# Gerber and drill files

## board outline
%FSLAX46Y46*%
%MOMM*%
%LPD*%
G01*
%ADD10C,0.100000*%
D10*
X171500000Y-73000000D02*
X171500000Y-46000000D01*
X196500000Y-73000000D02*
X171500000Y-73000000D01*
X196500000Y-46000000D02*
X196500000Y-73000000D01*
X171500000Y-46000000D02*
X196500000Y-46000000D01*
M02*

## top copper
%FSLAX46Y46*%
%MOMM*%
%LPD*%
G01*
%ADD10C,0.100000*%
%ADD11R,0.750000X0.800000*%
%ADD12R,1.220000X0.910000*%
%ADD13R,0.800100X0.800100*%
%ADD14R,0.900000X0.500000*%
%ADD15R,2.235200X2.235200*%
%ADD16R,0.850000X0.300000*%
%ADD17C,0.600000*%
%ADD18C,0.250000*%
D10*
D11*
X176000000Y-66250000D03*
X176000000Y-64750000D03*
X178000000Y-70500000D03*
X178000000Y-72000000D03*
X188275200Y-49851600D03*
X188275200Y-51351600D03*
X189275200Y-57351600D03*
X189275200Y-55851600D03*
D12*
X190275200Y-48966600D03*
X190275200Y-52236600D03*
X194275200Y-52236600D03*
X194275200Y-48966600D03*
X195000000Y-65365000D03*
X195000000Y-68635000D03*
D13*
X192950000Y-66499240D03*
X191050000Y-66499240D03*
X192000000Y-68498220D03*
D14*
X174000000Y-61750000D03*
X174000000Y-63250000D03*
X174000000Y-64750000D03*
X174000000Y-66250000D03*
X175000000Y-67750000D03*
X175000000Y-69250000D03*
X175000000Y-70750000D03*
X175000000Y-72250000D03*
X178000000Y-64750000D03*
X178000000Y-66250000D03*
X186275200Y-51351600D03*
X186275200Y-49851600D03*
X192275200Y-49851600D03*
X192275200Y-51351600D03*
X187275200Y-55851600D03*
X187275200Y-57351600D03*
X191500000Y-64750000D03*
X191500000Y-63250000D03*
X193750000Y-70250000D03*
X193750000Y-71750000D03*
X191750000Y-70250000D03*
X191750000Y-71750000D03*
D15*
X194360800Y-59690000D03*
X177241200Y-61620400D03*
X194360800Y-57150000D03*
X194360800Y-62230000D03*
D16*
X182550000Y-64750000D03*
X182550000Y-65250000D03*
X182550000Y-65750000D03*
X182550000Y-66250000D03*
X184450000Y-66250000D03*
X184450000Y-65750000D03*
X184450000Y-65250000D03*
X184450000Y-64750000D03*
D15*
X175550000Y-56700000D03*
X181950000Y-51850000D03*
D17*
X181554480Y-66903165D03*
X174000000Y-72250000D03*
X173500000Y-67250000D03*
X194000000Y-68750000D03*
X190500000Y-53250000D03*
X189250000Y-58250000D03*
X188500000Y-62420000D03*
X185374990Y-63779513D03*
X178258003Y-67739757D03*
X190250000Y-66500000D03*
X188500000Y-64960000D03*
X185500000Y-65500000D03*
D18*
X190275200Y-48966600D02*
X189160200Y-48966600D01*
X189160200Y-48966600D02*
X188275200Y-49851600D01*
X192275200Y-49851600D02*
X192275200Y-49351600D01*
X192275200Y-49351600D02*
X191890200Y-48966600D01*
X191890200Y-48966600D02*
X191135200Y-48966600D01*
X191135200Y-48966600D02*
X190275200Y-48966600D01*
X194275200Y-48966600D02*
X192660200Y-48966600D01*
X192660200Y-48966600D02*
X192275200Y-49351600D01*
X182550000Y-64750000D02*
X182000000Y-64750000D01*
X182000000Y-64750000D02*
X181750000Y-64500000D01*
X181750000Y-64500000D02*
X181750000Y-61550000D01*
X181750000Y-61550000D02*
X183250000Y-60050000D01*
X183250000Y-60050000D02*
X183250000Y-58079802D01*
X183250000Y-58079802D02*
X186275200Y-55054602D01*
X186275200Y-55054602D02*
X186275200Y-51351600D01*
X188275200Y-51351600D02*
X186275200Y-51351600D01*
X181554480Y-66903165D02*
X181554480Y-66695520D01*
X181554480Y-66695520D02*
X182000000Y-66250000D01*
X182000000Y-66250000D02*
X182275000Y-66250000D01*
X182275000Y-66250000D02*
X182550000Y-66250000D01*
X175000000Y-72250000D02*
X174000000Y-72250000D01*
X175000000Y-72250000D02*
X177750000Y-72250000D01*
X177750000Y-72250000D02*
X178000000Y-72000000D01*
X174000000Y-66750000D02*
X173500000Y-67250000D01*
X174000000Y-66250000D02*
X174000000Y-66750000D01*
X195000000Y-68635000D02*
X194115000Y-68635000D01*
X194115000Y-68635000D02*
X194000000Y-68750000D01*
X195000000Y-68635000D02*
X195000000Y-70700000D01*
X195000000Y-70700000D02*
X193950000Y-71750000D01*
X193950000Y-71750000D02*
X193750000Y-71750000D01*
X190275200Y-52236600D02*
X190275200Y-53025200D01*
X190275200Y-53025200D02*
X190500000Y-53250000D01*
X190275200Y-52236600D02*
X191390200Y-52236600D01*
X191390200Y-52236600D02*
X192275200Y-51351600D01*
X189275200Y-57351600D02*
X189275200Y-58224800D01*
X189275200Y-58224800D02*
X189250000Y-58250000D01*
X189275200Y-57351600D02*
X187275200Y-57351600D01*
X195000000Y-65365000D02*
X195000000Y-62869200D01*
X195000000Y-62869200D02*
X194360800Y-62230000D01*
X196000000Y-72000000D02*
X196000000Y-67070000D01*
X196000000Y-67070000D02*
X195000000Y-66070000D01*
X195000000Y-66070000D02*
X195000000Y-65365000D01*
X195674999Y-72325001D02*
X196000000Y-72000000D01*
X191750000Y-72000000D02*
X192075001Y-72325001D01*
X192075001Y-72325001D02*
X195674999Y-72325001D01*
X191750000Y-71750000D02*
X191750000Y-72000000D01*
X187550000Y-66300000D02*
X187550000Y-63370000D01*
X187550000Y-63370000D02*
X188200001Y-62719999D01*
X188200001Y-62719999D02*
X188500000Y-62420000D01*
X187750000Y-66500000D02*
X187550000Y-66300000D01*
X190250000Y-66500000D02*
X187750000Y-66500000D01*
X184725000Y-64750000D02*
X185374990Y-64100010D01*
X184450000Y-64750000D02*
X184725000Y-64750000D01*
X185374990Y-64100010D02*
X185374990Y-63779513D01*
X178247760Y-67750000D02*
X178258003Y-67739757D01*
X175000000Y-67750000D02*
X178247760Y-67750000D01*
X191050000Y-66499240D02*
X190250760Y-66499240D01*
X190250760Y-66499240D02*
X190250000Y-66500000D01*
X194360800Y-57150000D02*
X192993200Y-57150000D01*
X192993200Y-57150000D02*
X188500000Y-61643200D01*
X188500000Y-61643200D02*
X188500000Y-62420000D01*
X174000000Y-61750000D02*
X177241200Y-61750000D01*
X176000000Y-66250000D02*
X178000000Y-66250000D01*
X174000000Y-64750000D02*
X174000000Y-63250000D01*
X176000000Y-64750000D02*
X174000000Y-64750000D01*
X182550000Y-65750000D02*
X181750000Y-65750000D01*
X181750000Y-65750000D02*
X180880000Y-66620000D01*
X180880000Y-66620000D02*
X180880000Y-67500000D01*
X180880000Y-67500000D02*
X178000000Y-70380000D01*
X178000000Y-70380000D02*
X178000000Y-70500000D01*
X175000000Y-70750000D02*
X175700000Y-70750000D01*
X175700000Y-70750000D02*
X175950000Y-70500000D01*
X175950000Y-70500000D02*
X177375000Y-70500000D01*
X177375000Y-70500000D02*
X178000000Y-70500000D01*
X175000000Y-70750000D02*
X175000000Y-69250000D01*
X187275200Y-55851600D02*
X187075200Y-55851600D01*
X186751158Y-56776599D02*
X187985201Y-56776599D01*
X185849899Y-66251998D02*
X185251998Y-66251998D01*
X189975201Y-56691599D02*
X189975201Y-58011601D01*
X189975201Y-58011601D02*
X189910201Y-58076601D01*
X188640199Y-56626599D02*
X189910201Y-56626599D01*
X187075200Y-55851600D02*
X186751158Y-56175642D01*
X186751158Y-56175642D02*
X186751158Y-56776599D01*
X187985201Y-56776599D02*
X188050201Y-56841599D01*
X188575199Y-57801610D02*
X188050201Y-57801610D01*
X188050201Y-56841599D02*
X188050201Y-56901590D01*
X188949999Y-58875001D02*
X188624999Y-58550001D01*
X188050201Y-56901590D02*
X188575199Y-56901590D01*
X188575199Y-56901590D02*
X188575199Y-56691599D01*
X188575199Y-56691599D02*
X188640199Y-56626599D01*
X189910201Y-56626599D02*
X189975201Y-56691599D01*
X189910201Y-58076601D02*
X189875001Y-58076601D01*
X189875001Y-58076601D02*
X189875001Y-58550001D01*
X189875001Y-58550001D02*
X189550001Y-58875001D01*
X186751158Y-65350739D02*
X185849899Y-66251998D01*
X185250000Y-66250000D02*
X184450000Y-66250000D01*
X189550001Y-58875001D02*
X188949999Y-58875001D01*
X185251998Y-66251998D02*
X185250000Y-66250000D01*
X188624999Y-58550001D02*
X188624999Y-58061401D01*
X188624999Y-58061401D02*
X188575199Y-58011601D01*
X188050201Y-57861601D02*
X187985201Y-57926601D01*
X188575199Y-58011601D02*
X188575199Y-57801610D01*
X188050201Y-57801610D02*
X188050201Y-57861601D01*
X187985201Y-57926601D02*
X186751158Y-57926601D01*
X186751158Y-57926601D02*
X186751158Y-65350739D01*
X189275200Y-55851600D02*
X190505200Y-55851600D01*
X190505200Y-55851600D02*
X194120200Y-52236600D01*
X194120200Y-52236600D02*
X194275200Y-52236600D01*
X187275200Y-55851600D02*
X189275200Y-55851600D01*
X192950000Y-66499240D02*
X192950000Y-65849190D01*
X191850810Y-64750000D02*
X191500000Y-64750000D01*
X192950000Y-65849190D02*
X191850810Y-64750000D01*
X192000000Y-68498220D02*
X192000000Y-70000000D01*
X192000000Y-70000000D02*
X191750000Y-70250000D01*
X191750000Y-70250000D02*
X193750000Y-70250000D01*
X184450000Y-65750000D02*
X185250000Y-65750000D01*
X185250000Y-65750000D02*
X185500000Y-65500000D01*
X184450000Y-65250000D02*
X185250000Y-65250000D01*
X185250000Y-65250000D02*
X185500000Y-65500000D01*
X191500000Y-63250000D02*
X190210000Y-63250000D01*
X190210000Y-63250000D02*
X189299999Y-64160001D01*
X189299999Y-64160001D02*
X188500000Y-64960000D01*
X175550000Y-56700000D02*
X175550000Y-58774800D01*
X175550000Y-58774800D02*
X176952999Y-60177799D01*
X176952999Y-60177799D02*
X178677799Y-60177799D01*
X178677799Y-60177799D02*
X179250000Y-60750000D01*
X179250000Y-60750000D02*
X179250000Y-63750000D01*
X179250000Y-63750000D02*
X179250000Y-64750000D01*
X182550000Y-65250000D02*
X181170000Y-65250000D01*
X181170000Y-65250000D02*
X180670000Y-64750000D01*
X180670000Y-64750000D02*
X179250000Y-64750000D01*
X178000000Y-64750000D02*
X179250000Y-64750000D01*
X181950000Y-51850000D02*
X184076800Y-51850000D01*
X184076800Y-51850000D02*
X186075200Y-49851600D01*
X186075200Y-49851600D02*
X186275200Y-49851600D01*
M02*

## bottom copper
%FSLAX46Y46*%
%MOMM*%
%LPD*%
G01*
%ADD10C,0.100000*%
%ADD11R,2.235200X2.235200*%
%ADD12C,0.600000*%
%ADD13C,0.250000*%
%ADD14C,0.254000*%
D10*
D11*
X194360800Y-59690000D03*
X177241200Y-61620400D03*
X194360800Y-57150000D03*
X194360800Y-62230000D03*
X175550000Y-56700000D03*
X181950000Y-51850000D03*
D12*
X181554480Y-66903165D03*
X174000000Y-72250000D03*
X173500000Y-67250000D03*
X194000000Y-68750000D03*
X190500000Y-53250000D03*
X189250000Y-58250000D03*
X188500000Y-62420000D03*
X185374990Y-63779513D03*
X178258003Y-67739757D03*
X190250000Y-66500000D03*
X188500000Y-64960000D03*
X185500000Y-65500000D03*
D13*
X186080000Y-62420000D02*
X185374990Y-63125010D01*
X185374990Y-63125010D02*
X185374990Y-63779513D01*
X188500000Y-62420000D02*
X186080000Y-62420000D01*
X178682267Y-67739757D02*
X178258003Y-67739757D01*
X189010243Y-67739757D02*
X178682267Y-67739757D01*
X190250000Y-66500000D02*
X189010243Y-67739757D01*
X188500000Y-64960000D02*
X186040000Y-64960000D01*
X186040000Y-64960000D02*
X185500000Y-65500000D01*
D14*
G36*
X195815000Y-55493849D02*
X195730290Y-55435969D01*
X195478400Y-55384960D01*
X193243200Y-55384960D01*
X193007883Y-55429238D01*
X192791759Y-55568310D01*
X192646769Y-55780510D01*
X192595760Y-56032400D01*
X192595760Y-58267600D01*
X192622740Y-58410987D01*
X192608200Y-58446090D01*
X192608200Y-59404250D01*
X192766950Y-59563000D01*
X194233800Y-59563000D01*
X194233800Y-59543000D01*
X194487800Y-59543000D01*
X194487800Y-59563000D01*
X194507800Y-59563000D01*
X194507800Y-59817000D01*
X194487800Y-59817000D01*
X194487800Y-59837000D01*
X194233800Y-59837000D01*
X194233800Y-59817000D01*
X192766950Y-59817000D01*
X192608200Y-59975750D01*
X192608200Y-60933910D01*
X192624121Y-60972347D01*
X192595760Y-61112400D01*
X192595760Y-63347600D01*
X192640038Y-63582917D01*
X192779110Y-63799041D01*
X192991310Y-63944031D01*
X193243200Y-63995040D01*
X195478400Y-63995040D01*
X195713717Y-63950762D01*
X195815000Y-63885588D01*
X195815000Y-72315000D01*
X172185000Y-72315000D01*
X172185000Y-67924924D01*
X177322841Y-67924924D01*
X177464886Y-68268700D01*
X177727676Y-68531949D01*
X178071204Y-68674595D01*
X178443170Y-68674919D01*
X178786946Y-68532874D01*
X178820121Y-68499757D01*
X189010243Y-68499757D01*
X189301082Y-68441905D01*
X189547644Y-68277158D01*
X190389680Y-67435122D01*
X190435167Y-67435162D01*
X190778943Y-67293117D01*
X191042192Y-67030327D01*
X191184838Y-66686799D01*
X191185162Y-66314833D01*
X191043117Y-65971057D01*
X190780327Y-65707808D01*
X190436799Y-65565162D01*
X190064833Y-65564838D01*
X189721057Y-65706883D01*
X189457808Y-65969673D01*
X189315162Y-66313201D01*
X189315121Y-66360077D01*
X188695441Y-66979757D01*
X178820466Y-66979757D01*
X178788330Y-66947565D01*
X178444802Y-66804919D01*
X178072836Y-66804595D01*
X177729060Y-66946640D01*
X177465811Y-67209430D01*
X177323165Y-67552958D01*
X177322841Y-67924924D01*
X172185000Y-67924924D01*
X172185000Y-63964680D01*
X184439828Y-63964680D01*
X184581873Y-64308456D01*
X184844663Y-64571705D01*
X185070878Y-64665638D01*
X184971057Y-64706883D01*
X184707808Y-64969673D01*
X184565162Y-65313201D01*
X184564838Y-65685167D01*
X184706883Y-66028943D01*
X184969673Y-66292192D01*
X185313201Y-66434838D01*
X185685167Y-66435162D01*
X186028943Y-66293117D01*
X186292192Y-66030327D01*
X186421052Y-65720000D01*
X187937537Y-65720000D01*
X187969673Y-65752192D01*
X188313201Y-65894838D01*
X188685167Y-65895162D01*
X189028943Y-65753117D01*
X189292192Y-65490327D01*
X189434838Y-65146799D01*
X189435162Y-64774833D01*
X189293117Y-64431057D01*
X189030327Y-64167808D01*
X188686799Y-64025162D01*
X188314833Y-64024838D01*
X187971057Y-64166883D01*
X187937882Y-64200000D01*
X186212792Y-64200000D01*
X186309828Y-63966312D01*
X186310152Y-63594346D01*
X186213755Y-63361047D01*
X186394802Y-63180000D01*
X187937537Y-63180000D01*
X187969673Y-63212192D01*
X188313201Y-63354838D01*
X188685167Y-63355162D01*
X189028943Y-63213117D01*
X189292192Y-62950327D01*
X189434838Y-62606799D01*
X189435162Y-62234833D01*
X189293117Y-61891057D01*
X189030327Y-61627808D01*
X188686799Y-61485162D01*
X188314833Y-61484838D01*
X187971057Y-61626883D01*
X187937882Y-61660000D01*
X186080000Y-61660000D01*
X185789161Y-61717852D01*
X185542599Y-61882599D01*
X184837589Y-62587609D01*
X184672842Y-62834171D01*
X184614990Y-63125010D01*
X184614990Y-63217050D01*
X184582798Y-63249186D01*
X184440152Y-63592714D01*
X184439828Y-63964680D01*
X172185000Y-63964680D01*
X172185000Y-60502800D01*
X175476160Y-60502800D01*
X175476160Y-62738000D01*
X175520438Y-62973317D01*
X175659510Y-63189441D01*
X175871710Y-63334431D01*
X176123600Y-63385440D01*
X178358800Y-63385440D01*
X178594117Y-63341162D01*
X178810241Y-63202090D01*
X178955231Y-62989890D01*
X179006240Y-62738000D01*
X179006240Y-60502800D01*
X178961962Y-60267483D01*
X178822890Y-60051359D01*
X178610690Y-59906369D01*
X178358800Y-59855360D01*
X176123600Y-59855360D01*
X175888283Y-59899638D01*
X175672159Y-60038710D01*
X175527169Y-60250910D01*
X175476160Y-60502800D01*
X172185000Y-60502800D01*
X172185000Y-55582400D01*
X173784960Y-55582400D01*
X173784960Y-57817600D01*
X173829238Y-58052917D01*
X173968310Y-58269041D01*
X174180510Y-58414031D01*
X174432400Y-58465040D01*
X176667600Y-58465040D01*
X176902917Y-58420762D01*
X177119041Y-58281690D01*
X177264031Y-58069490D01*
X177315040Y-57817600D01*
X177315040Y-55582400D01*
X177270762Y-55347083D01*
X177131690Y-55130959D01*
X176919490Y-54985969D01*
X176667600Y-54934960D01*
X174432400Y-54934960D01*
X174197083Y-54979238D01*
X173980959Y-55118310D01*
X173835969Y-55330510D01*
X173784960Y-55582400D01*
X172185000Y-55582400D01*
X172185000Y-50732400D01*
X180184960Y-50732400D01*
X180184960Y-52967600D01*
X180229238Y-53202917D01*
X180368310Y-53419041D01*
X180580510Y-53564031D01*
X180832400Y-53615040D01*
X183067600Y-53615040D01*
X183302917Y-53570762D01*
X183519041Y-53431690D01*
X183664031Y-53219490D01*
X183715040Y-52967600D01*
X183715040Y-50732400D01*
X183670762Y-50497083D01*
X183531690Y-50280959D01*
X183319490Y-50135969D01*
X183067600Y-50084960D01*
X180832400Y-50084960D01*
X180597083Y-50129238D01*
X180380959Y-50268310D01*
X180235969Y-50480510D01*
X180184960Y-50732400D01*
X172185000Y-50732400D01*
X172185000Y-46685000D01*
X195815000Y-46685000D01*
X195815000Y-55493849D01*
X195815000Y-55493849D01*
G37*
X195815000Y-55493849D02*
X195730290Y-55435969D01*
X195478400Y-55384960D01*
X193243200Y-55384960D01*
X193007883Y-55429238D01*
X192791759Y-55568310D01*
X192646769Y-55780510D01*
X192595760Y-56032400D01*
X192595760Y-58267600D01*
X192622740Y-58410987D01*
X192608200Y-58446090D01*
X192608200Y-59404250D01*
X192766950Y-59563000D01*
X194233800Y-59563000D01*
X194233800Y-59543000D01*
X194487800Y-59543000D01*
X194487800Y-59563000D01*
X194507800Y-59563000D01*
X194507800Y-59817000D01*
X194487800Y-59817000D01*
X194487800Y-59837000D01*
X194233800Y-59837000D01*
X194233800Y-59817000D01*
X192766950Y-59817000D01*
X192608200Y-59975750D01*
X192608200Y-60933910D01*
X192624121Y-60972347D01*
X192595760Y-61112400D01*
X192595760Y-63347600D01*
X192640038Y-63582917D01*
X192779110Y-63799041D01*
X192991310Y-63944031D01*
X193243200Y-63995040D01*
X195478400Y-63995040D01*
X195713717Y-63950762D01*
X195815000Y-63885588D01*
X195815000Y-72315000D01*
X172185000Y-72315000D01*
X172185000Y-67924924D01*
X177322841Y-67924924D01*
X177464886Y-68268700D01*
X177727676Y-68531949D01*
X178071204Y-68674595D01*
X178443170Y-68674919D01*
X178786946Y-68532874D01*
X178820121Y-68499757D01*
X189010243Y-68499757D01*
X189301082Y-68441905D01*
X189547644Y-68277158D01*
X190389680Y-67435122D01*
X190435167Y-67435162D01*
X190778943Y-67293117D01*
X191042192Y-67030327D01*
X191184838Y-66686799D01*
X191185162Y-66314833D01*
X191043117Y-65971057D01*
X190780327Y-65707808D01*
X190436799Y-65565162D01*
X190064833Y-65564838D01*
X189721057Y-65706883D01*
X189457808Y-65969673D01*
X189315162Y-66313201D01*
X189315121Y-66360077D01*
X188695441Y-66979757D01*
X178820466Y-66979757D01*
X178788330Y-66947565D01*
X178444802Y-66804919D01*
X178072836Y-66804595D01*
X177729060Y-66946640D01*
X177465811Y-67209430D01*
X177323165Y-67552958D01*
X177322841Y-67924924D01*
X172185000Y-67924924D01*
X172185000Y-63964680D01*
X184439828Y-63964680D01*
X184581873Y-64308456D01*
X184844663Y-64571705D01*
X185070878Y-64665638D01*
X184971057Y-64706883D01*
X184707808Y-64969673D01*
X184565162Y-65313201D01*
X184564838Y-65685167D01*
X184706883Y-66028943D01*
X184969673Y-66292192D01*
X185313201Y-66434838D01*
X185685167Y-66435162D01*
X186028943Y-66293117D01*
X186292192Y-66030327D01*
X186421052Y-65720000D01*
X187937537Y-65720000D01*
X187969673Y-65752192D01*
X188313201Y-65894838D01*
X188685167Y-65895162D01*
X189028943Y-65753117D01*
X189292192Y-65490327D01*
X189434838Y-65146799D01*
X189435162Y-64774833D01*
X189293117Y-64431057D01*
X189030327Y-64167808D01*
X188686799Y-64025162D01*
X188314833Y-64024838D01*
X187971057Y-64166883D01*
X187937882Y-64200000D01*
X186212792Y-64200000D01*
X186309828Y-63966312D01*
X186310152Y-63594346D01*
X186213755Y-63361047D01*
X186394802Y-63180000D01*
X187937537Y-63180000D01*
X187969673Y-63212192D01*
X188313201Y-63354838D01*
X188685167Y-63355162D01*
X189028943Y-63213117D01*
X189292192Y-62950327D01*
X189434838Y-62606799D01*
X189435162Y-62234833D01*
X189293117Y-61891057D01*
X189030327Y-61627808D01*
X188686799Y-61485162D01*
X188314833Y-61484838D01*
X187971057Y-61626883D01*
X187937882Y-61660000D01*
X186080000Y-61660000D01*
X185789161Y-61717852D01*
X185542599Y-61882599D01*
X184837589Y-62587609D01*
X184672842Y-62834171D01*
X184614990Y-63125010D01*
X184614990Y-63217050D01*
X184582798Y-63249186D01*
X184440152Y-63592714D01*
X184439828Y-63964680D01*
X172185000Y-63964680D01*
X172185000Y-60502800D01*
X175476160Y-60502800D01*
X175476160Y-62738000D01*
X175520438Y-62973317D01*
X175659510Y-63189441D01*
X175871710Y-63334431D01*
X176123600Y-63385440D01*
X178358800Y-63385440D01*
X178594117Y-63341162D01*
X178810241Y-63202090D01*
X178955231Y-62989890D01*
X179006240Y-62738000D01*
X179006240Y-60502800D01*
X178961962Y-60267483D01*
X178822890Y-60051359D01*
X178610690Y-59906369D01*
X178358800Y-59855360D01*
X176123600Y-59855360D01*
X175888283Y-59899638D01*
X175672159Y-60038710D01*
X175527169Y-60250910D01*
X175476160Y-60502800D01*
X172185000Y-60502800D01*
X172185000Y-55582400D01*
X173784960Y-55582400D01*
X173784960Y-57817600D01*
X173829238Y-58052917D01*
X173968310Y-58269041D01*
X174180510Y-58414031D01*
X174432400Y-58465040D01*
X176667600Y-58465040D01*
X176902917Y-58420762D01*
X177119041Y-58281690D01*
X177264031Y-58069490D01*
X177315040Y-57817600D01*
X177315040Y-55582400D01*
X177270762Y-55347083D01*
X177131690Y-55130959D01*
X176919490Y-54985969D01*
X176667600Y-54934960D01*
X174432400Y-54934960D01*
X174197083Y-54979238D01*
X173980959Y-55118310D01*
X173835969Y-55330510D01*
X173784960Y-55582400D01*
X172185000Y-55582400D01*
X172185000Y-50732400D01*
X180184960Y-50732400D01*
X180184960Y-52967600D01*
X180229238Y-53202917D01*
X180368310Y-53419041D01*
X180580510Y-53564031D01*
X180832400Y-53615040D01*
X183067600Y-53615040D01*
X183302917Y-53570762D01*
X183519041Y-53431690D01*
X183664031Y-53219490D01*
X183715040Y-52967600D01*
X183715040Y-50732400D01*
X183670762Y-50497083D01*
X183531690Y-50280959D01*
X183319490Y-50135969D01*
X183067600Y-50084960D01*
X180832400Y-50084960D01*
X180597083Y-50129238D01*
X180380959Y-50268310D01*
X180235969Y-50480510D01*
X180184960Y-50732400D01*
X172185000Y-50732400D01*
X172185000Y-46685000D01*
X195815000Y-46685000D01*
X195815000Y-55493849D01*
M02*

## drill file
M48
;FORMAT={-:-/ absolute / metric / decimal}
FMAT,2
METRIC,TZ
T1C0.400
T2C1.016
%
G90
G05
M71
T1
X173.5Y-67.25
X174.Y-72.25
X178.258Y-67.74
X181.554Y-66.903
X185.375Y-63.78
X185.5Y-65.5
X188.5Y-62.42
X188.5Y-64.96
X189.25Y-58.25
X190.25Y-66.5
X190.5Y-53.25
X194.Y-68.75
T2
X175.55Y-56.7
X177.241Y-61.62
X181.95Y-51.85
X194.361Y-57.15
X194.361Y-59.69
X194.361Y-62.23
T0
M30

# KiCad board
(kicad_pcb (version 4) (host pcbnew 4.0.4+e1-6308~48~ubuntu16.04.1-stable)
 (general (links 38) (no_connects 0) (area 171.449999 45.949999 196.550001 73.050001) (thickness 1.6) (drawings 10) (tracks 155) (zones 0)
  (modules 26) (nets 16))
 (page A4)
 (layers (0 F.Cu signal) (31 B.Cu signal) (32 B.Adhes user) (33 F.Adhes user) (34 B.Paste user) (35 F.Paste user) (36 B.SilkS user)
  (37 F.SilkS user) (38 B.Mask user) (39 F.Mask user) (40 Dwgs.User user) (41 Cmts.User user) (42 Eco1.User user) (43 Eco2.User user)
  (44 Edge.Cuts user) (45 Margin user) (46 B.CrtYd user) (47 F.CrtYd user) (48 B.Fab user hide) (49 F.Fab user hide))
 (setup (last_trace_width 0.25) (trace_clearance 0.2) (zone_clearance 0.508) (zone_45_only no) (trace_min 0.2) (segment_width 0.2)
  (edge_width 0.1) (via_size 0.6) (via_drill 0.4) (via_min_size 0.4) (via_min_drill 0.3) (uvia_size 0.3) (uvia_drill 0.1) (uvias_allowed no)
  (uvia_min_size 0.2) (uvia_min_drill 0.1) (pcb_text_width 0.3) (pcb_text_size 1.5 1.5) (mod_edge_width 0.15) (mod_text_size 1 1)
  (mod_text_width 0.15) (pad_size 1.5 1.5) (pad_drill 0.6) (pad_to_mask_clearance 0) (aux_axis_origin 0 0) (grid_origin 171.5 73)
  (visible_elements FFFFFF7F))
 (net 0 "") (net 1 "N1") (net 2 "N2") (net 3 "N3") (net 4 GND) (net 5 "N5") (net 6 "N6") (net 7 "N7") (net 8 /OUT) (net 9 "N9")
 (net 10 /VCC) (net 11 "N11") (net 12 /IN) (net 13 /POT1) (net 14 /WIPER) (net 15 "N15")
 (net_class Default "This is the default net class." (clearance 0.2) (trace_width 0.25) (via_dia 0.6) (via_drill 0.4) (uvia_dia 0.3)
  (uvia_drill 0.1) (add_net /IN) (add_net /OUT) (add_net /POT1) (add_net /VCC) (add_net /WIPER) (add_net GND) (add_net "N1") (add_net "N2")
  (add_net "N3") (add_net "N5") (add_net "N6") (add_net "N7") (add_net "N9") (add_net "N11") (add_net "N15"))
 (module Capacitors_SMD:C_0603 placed (layer F.Cu) (at 176 65.5 90)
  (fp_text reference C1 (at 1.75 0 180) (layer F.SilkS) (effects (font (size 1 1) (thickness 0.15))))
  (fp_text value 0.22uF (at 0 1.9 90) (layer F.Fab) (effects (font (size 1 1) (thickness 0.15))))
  (pad 1 smd rect (at -0.75 0 90) (size 0.8 0.75) (layers F.Cu F.Paste F.Mask) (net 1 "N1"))
  (pad 2 smd rect (at 0.75 0 90) (size 0.8 0.75) (layers F.Cu F.Paste F.Mask) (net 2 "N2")))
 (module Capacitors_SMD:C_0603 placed (layer F.Cu) (at 178 71.25 270)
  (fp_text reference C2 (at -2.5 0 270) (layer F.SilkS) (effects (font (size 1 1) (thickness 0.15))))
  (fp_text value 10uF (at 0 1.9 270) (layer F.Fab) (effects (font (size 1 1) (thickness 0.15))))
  (pad 1 smd rect (at -0.75 0 270) (size 0.8 0.75) (layers F.Cu F.Paste F.Mask) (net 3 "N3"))
  (pad 2 smd rect (at 0.75 0 270) (size 0.8 0.75) (layers F.Cu F.Paste F.Mask) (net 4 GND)))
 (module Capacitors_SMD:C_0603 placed (layer F.Cu) (at 188.2752 50.6016 270)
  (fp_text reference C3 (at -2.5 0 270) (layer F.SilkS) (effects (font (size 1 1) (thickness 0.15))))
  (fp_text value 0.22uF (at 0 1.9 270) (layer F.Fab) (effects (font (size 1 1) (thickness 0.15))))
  (pad 1 smd rect (at -0.75 0 270) (size 0.8 0.75) (layers F.Cu F.Paste F.Mask) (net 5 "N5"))
  (pad 2 smd rect (at 0.75 0 270) (size 0.8 0.75) (layers F.Cu F.Paste F.Mask) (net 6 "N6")))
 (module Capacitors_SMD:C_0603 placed (layer F.Cu) (at 189.2752 56.6016 90)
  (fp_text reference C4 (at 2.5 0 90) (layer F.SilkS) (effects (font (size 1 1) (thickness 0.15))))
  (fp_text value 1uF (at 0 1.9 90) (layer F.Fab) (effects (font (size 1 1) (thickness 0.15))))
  (pad 1 smd rect (at -0.75 0 90) (size 0.8 0.75) (layers F.Cu F.Paste F.Mask) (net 4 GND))
  (pad 2 smd rect (at 0.75 0 90) (size 0.8 0.75) (layers F.Cu F.Paste F.Mask) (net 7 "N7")))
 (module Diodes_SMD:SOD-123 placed (layer F.Cu) (at 190.2752 50.6016 270)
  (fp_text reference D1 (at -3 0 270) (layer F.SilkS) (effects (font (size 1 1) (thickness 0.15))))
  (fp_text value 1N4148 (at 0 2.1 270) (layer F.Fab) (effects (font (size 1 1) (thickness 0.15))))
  (pad 1 smd rect (at -1.635 0 270) (size 0.91 1.22) (layers F.Cu F.Paste F.Mask) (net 5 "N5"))
  (pad 2 smd rect (at 1.635 0 270) (size 0.91 1.22) (layers F.Cu F.Paste F.Mask) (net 4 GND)))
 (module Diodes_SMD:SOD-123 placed (layer F.Cu) (at 194.2752 50.6016 90)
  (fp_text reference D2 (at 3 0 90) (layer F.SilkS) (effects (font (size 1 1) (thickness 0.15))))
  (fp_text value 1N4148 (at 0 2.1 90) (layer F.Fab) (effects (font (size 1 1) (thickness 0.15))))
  (pad 1 smd rect (at -1.635 0 90) (size 0.91 1.22) (layers F.Cu F.Paste F.Mask) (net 7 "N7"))
  (pad 2 smd rect (at 1.635 0 90) (size 0.91 1.22) (layers F.Cu F.Paste F.Mask) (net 5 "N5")))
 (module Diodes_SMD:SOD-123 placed (layer F.Cu) (at 195 67 270)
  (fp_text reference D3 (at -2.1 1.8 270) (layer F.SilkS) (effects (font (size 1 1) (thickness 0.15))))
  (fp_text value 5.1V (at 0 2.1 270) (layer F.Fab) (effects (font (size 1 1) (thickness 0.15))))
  (pad 1 smd rect (at -1.635 0 270) (size 0.91 1.22) (layers F.Cu F.Paste F.Mask) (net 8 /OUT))
  (pad 2 smd rect (at 1.635 0 270) (size 0.91 1.22) (layers F.Cu F.Paste F.Mask) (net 4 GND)))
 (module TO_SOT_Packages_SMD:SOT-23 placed (layer F.Cu) (at 192 67.5 180)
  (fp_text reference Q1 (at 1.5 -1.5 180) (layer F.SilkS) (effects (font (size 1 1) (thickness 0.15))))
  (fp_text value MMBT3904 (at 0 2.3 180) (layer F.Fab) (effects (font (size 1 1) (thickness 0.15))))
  (pad 1 smd rect (at -0.95 1.00076 180) (size 0.8001 0.8001) (layers F.Cu F.Paste F.Mask) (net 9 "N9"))
  (pad 2 smd rect (at 0.95 1.00076 180) (size 0.8001 0.8001) (layers F.Cu F.Paste F.Mask) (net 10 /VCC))
  (pad 3 smd rect (at 0 -0.99822 180) (size 0.8001 0.8001) (layers F.Cu F.Paste F.Mask) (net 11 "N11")))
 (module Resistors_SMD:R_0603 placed (layer F.Cu) (at 174 62.5 270)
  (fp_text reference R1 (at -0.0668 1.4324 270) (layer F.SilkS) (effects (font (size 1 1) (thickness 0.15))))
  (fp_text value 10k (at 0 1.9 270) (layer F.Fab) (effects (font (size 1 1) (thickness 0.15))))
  (pad 1 smd rect (at -0.75 0 270) (size 0.5 0.9) (layers F.Cu F.Paste F.Mask) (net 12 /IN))
  (pad 2 smd rect (at 0.75 0 270) (size 0.5 0.9) (layers F.Cu F.Paste F.Mask) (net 2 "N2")))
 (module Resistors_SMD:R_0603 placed (layer F.Cu) (at 174 65.5 270)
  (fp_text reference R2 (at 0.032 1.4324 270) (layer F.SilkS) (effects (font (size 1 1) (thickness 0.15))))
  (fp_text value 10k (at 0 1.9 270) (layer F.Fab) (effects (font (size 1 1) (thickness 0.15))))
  (pad 1 smd rect (at -0.75 0 270) (size 0.5 0.9) (layers F.Cu F.Paste F.Mask) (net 2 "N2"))
  (pad 2 smd rect (at 0.75 0 270) (size 0.5 0.9) (layers F.Cu F.Paste F.Mask) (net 4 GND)))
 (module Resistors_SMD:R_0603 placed (layer F.Cu) (at 175 68.5 270)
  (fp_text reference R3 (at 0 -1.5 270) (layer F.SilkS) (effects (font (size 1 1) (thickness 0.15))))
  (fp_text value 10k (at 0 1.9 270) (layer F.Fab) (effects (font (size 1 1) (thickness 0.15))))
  (pad 1 smd rect (at -0.75 0 270) (size 0.5 0.9) (layers F.Cu F.Paste F.Mask) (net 10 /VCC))
  (pad 2 smd rect (at 0.75 0 270) (size 0.5 0.9) (layers F.Cu F.Paste F.Mask) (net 3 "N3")))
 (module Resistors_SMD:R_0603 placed (layer F.Cu) (at 175 71.5 270)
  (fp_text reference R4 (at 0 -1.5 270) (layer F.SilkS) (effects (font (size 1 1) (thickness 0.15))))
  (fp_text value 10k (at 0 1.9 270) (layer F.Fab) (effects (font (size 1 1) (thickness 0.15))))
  (pad 1 smd rect (at -0.75 0 270) (size 0.5 0.9) (layers F.Cu F.Paste F.Mask) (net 3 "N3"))
  (pad 2 smd rect (at 0.75 0 270) (size 0.5 0.9) (layers F.Cu F.Paste F.Mask) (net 4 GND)))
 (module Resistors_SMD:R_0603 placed (layer F.Cu) (at 178 65.5 270)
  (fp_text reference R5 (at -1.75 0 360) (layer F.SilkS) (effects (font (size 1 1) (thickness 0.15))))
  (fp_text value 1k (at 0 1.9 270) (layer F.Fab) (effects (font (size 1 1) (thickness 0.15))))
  (pad 1 smd rect (at -0.75 0 270) (size 0.5 0.9) (layers F.Cu F.Paste F.Mask) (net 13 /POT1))
  (pad 2 smd rect (at 0.75 0 270) (size 0.5 0.9) (layers F.Cu F.Paste F.Mask) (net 1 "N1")))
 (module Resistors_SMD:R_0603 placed (layer F.Cu) (at 186.2752 50.6016 90)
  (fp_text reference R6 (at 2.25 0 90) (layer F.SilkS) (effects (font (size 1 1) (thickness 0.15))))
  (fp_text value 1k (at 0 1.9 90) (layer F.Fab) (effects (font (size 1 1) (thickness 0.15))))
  (pad 1 smd rect (at -0.75 0 90) (size 0.5 0.9) (layers F.Cu F.Paste F.Mask) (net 6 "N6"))
  (pad 2 smd rect (at 0.75 0 90) (size 0.5 0.9) (layers F.Cu F.Paste F.Mask) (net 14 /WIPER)))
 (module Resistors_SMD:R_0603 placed (layer F.Cu) (at 192.2752 50.6016 270)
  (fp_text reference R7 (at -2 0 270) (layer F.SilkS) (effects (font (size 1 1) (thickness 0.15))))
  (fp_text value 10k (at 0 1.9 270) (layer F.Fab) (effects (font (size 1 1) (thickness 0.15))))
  (pad 1 smd rect (at -0.75 0 270) (size 0.5 0.9) (layers F.Cu F.Paste F.Mask) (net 5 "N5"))
  (pad 2 smd rect (at 0.75 0 270) (size 0.5 0.9) (layers F.Cu F.Paste F.Mask) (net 4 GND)))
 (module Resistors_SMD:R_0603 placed (layer F.Cu) (at 187.2752 56.6016 270)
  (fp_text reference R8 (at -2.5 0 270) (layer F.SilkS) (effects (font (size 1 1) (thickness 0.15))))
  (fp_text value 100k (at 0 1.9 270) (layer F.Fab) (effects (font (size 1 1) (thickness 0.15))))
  (pad 1 smd rect (at -0.75 0 270) (size 0.5 0.9) (layers F.Cu F.Paste F.Mask) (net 7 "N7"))
  (pad 2 smd rect (at 0.75 0 270) (size 0.5 0.9) (layers F.Cu F.Paste F.Mask) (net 4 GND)))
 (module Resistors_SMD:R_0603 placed (layer F.Cu) (at 191.5 64 90)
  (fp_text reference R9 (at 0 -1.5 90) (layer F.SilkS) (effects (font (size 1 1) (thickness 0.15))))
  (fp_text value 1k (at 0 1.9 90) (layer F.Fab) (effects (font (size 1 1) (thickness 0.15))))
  (pad 1 smd rect (at -0.75 0 90) (size 0.5 0.9) (layers F.Cu F.Paste F.Mask) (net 9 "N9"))
  (pad 2 smd rect (at 0.75 0 90) (size 0.5 0.9) (layers F.Cu F.Paste F.Mask) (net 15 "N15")))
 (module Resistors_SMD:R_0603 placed (layer F.Cu) (at 193.75 71 270)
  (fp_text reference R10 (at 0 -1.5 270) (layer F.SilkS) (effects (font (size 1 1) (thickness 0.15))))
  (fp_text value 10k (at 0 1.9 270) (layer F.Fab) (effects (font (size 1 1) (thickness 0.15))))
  (pad 1 smd rect (at -0.75 0 270) (size 0.5 0.9) (layers F.Cu F.Paste F.Mask) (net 11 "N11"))
  (pad 2 smd rect (at 0.75 0 270) (size 0.5 0.9) (layers F.Cu F.Paste F.Mask) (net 4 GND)))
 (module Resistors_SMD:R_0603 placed (layer F.Cu) (at 191.75 71 270)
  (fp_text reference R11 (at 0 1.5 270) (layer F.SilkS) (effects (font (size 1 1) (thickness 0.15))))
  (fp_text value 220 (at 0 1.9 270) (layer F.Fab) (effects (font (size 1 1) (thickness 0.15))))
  (pad 1 smd rect (at -0.75 0 270) (size 0.5 0.9) (layers F.Cu F.Paste F.Mask) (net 11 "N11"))
  (pad 2 smd rect (at 0.75 0 270) (size 0.5 0.9) (layers F.Cu F.Paste F.Mask) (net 8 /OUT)))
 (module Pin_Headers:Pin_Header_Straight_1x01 (layer F.Cu) (at 194.3608 59.69)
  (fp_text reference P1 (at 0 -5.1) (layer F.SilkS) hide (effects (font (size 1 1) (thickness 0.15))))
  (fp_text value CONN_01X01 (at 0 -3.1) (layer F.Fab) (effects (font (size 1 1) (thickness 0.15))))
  (pad 1 thru_hole rect (at 0 0) (size 2.2352 2.2352) (drill 1.016) (layers *.Cu *.Mask F.SilkS) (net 4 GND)))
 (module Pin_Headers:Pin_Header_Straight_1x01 (layer F.Cu) (at 177.2412 61.6204)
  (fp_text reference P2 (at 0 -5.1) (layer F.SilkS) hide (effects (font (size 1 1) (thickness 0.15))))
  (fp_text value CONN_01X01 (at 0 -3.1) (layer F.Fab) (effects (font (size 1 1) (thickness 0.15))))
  (pad 1 thru_hole rect (at 0 0) (size 2.2352 2.2352) (drill 1.016) (layers *.Cu *.Mask F.SilkS) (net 12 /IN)))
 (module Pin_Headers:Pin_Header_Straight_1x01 (layer F.Cu) (at 194.3608 57.15)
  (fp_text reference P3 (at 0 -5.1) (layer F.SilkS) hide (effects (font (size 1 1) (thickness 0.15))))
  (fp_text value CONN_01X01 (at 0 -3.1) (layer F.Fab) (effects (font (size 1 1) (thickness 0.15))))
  (pad 1 thru_hole rect (at 0 0) (size 2.2352 2.2352) (drill 1.016) (layers *.Cu *.Mask F.SilkS) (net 10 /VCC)))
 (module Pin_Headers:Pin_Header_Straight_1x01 (layer F.Cu) (at 194.3608 62.23)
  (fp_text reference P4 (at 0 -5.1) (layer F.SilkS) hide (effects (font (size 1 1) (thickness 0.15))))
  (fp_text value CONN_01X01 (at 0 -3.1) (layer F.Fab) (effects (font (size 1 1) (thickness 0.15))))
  (pad 1 thru_hole rect (at 0 0) (size 2.2352 2.2352) (drill 1.016) (layers *.Cu *.Mask F.SilkS) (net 8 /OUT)))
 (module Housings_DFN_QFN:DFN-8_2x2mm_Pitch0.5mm (layer F.Cu) (at 183.5 65.5)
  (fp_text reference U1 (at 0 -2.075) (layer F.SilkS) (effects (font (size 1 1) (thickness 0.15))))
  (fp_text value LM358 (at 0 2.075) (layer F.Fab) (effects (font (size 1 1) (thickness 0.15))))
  (pad 1 smd rect (at -0.95 -0.75) (size 0.85 0.3) (layers F.Cu F.Paste F.Mask) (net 6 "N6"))
  (pad 2 smd rect (at -0.95 -0.25) (size 0.85 0.3) (layers F.Cu F.Paste F.Mask) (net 13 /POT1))
  (pad 3 smd rect (at -0.95 0.25) (size 0.85 0.3) (layers F.Cu F.Paste F.Mask) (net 3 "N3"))
  (pad 4 smd rect (at -0.95 0.75) (size 0.85 0.3) (layers F.Cu F.Paste F.Mask) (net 4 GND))
  (pad 5 smd rect (at 0.95 0.75) (size 0.85 0.3) (layers F.Cu F.Paste F.Mask) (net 7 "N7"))
  (pad 6 smd rect (at 0.95 0.25) (size 0.85 0.3) (layers F.Cu F.Paste F.Mask) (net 15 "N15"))
  (pad 7 smd rect (at 0.95 -0.25) (size 0.85 0.3) (layers F.Cu F.Paste F.Mask) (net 15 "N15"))
  (pad 8 smd rect (at 0.95 -0.75) (size 0.85 0.3) (layers F.Cu F.Paste F.Mask) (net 10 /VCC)))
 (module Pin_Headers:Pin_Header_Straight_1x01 (layer F.Cu) (at 175.55 56.7)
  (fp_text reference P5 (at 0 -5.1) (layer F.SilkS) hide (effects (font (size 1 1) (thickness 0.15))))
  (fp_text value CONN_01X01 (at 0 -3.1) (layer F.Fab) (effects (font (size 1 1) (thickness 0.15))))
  (pad 1 thru_hole rect (at 0 0) (size 2.2352 2.2352) (drill 1.016) (layers *.Cu *.Mask F.SilkS) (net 13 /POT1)))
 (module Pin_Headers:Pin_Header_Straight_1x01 (layer F.Cu) (at 181.95 51.85)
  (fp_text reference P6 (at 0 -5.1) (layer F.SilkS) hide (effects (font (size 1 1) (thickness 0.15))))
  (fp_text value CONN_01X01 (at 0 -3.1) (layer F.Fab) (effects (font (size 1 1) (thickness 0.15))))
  (pad 1 thru_hole rect (at 0 0) (size 2.2352 2.2352) (drill 1.016) (layers *.Cu *.Mask F.SilkS) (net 14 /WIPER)))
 (gr_line (start 171.5 73) (end 171.5 46) (layer Edge.Cuts) (width 0.1))
 (gr_line (start 196.5 73) (end 171.5 73) (layer Edge.Cuts) (width 0.1))
 (gr_line (start 196.5 46) (end 196.5 73) (layer Edge.Cuts) (width 0.1))
 (gr_line (start 171.5 46) (end 196.5 46) (layer Edge.Cuts) (width 0.1))
 (segment (start 190.2752 48.9666) (end 189.1602 48.9666) (width 0.25) (layer F.Cu) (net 5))
 (segment (start 189.1602 48.9666) (end 188.2752 49.8516) (width 0.25) (layer F.Cu) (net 5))
 (segment (start 192.2752 49.8516) (end 192.2752 49.3516) (width 0.25) (layer F.Cu) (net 5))
 (segment (start 192.2752 49.3516) (end 191.8902 48.9666) (width 0.25) (layer F.Cu) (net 5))
 (segment (start 191.8902 48.9666) (end 191.1352 48.9666) (width 0.25) (layer F.Cu) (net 5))
 (segment (start 191.1352 48.9666) (end 190.2752 48.9666) (width 0.25) (layer F.Cu) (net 5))
 (segment (start 194.2752 48.9666) (end 192.6602 48.9666) (width 0.25) (layer F.Cu) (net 5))
 (segment (start 192.6602 48.9666) (end 192.2752 49.3516) (width 0.25) (layer F.Cu) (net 5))
 (segment (start 182.55 64.75) (end 182 64.75) (width 0.25) (layer F.Cu) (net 6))
 (segment (start 182 64.75) (end 181.75 64.5) (width 0.25) (layer F.Cu) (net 6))
 (segment (start 181.75 64.5) (end 181.75 61.55) (width 0.25) (layer F.Cu) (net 6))
 (segment (start 181.75 61.55) (end 183.25 60.05) (width 0.25) (layer F.Cu) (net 6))
 (segment (start 183.25 60.05) (end 183.25 58.079802) (width 0.25) (layer F.Cu) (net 6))
 (segment (start 183.25 58.079802) (end 186.2752 55.054602) (width 0.25) (layer F.Cu) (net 6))
 (segment (start 186.2752 55.054602) (end 186.2752 51.3516) (width 0.25) (layer F.Cu) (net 6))
 (segment (start 188.2752 51.3516) (end 186.2752 51.3516) (width 0.25) (layer F.Cu) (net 6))
 (via (at 181.55448 66.903165) (size 0.6) (drill 0.4) (layers F.Cu B.Cu) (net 4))
 (segment (start 181.55448 66.903165) (end 181.55448 66.69552) (width 0.25) (layer F.Cu) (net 4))
 (segment (start 181.55448 66.69552) (end 182 66.25) (width 0.25) (layer F.Cu) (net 4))
 (segment (start 182 66.25) (end 182.275 66.25) (width 0.25) (layer F.Cu) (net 4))
 (segment (start 182.275 66.25) (end 182.55 66.25) (width 0.25) (layer F.Cu) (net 4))
 (segment (start 175 72.25) (end 174 72.25) (width 0.25) (layer F.Cu) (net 4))
 (via (at 174 72.25) (size 0.6) (drill 0.4) (layers F.Cu B.Cu) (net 4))
 (segment (start 175 72.25) (end 177.75 72.25) (width 0.25) (layer F.Cu) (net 4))
 (segment (start 177.75 72.25) (end 178 72) (width 0.25) (layer F.Cu) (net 4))
 (segment (start 174 66.75) (end 173.5 67.25) (width 0.25) (layer F.Cu) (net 4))
 (via (at 173.5 67.25) (size 0.6) (drill 0.4) (layers F.Cu B.Cu) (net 4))
 (segment (start 174 66.25) (end 174 66.75) (width 0.25) (layer F.Cu) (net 4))
 (segment (start 195 68.635) (end 194.115 68.635) (width 0.25) (layer F.Cu) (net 4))
 (segment (start 194.115 68.635) (end 194 68.75) (width 0.25) (layer F.Cu) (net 4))
 (via (at 194 68.75) (size 0.6) (drill 0.4) (layers F.Cu B.Cu) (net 4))
 (segment (start 195 68.635) (end 195 70.7) (width 0.25) (layer F.Cu) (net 4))
 (segment (start 195 70.7) (end 193.95 71.75) (width 0.25) (layer F.Cu) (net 4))
 (segment (start 193.95 71.75) (end 193.75 71.75) (width 0.25) (layer F.Cu) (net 4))
 (segment (start 190.2752 52.2366) (end 190.2752 53.0252) (width 0.25) (layer F.Cu) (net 4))
 (segment (start 190.2752 53.0252) (end 190.5 53.25) (width 0.25) (layer F.Cu) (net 4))
 (via (at 190.5 53.25) (size 0.6) (drill 0.4) (layers F.Cu B.Cu) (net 4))
 (segment (start 190.2752 52.2366) (end 191.3902 52.2366) (width 0.25) (layer F.Cu) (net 4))
 (segment (start 191.3902 52.2366) (end 192.2752 51.3516) (width 0.25) (layer F.Cu) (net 4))
 (segment (start 189.2752 57.3516) (end 189.2752 58.2248) (width 0.25) (layer F.Cu) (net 4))
 (segment (start 189.2752 58.2248) (end 189.25 58.25) (width 0.25) (layer F.Cu) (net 4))
 (via (at 189.25 58.25) (size 0.6) (drill 0.4) (layers F.Cu B.Cu) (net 4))
 (segment (start 189.2752 57.3516) (end 187.2752 57.3516) (width 0.25) (layer F.Cu) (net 4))
 (segment (start 195 65.365) (end 195 62.8692) (width 0.25) (layer F.Cu) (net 8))
 (segment (start 195 62.8692) (end 194.3608 62.23) (width 0.25) (layer F.Cu) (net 8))
 (segment (start 196 72) (end 196 67.07) (width 0.25) (layer F.Cu) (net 8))
 (segment (start 196 67.07) (end 195 66.07) (width 0.25) (layer F.Cu) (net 8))
 (segment (start 195 66.07) (end 195 65.365) (width 0.25) (layer F.Cu) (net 8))
 (segment (start 195.674999 72.325001) (end 196 72) (width 0.25) (layer F.Cu) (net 8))
 (segment (start 191.75 72) (end 192.075001 72.325001) (width 0.25) (layer F.Cu) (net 8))
 (segment (start 192.075001 72.325001) (end 195.674999 72.325001) (width 0.25) (layer F.Cu) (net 8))
 (segment (start 191.75 71.75) (end 191.75 72) (width 0.25) (layer F.Cu) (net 8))
 (segment (start 187.55 66.3) (end 187.55 63.37) (width 0.25) (layer F.Cu) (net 10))
 (segment (start 187.55 63.37) (end 188.200001 62.719999) (width 0.25) (layer F.Cu) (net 10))
 (segment (start 188.200001 62.719999) (end 188.5 62.42) (width 0.25) (layer F.Cu) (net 10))
 (segment (start 187.75 66.5) (end 187.55 66.3) (width 0.25) (layer F.Cu) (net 10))
 (segment (start 190.25 66.5) (end 187.75 66.5) (width 0.25) (layer F.Cu) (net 10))
 (segment (start 186.08 62.42) (end 185.37499 63.12501) (width 0.25) (layer B.Cu) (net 10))
 (segment (start 185.37499 63.12501) (end 185.37499 63.779513) (width 0.25) (layer B.Cu) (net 10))
 (segment (start 188.5 62.42) (end 186.08 62.42) (width 0.25) (layer B.Cu) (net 10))
 (via (at 188.5 62.42) (size 0.6) (drill 0.4) (layers F.Cu B.Cu) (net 10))
 (segment (start 184.725 64.75) (end 185.37499 64.10001) (width 0.25) (layer F.Cu) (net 10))
 (segment (start 184.45 64.75) (end 184.725 64.75) (width 0.25) (layer F.Cu) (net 10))
 (segment (start 185.37499 64.10001) (end 185.37499 63.779513) (width 0.25) (layer F.Cu) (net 10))
 (via (at 185.37499 63.779513) (size 0.6) (drill 0.4) (layers F.Cu B.Cu) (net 10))
 (segment (start 178.24776 67.75) (end 178.258003 67.739757) (width 0.25) (layer F.Cu) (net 10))
 (segment (start 175 67.75) (end 178.24776 67.75) (width 0.25) (layer F.Cu) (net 10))
 (segment (start 178.682267 67.739757) (end 178.258003 67.739757) (width 0.25) (layer B.Cu) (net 10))
 (segment (start 189.010243 67.739757) (end 178.682267 67.739757) (width 0.25) (layer B.Cu) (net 10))
 (segment (start 190.25 66.5) (end 189.010243 67.739757) (width 0.25) (layer B.Cu) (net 10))
 (via (at 178.258003 67.739757) (size 0.6) (drill 0.4) (layers F.Cu B.Cu) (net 10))
 (segment (start 191.05 66.49924) (end 190.25076 66.49924) (width 0.25) (layer F.Cu) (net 10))
 (segment (start 190.25076 66.49924) (end 190.25 66.5) (width 0.25) (layer F.Cu) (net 10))
 (via (at 190.25 66.5) (size 0.6) (drill 0.4) (layers F.Cu B.Cu) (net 10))
 (segment (start 194.3608 57.15) (end 192.9932 57.15) (width 0.25) (layer F.Cu) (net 10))
 (segment (start 192.9932 57.15) (end 188.5 61.6432) (width 0.25) (layer F.Cu) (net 10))
 (segment (start 188.5 61.6432) (end 188.5 62.42) (width 0.25) (layer F.Cu) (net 10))
 (segment (start 174 61.75) (end 177.2412 61.75) (width 0.25) (layer F.Cu) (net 12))
 (segment (start 176 66.25) (end 178 66.25) (width 0.25) (layer F.Cu) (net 1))
 (segment (start 174 64.75) (end 174 63.25) (width 0.25) (layer F.Cu) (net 2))
 (segment (start 176 64.75) (end 174 64.75) (width 0.25) (layer F.Cu) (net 2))
 (segment (start 182.55 65.75) (end 181.75 65.75) (width 0.25) (layer F.Cu) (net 3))
 (segment (start 181.75 65.75) (end 180.88 66.62) (width 0.25) (layer F.Cu) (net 3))
 (segment (start 180.88 66.62) (end 180.88 67.5) (width 0.25) (layer F.Cu) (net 3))
 (segment (start 180.88 67.5) (end 178 70.38) (width 0.25) (layer F.Cu) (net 3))
 (segment (start 178 70.38) (end 178 70.5) (width 0.25) (layer F.Cu) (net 3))
 (segment (start 175 70.75) (end 175.7 70.75) (width 0.25) (layer F.Cu) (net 3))
 (segment (start 175.7 70.75) (end 175.95 70.5) (width 0.25) (layer F.Cu) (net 3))
 (segment (start 175.95 70.5) (end 177.375 70.5) (width 0.25) (layer F.Cu) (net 3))
 (segment (start 177.375 70.5) (end 178 70.5) (width 0.25) (layer F.Cu) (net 3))
 (segment (start 175 70.75) (end 175 69.25) (width 0.25) (layer F.Cu) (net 3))
 (segment (start 187.2752 55.8516) (end 187.0752 55.8516) (width 0.25) (layer F.Cu) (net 7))
 (segment (start 186.751158 56.776599) (end 187.985201 56.776599) (width 0.25) (layer F.Cu) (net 7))
 (segment (start 185.849899 66.251998) (end 185.251998 66.251998) (width 0.25) (layer F.Cu) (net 7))
 (segment (start 189.975201 56.691599) (end 189.975201 58.011601) (width 0.25) (layer F.Cu) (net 7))
 (segment (start 189.975201 58.011601) (end 189.910201 58.076601) (width 0.25) (layer F.Cu) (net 7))
 (segment (start 188.640199 56.626599) (end 189.910201 56.626599) (width 0.25) (layer F.Cu) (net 7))
 (segment (start 187.0752 55.8516) (end 186.751158 56.175642) (width 0.25) (layer F.Cu) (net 7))
 (segment (start 186.751158 56.175642) (end 186.751158 56.776599) (width 0.25) (layer F.Cu) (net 7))
 (segment (start 187.985201 56.776599) (end 188.050201 56.841599) (width 0.25) (layer F.Cu) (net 7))
 (segment (start 188.575199 57.80161) (end 188.050201 57.80161) (width 0.25) (layer F.Cu) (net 7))
 (segment (start 188.050201 56.841599) (end 188.050201 56.90159) (width 0.25) (layer F.Cu) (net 7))
 (segment (start 188.949999 58.875001) (end 188.624999 58.550001) (width 0.25) (layer F.Cu) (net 7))
 (segment (start 188.050201 56.90159) (end 188.575199 56.90159) (width 0.25) (layer F.Cu) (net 7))
 (segment (start 188.575199 56.90159) (end 188.575199 56.691599) (width 0.25) (layer F.Cu) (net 7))
 (segment (start 188.575199 56.691599) (end 188.640199 56.626599) (width 0.25) (layer F.Cu) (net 7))
 (segment (start 189.910201 56.626599) (end 189.975201 56.691599) (width 0.25) (layer F.Cu) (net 7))
 (segment (start 189.910201 58.076601) (end 189.875001 58.076601) (width 0.25) (layer F.Cu) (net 7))
 (segment (start 189.875001 58.076601) (end 189.875001 58.550001) (width 0.25) (layer F.Cu) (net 7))
 (segment (start 189.875001 58.550001) (end 189.550001 58.875001) (width 0.25) (layer F.Cu) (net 7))
 (segment (start 186.751158 65.350739) (end 185.849899 66.251998) (width 0.25) (layer F.Cu) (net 7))
 (segment (start 185.25 66.25) (end 184.45 66.25) (width 0.25) (layer F.Cu) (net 7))
 (segment (start 189.550001 58.875001) (end 188.949999 58.875001) (width 0.25) (layer F.Cu) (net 7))
 (segment (start 185.251998 66.251998) (end 185.25 66.25) (width 0.25) (layer F.Cu) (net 7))
 (segment (start 188.624999 58.550001) (end 188.624999 58.061401) (width 0.25) (layer F.Cu) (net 7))
 (segment (start 188.624999 58.061401) (end 188.575199 58.011601) (width 0.25) (layer F.Cu) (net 7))
 (segment (start 188.050201 57.861601) (end 187.985201 57.926601) (width 0.25) (layer F.Cu) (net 7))
 (segment (start 188.575199 58.011601) (end 188.575199 57.80161) (width 0.25) (layer F.Cu) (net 7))
 (segment (start 188.050201 57.80161) (end 188.050201 57.861601) (width 0.25) (layer F.Cu) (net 7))
 (segment (start 187.985201 57.926601) (end 186.751158 57.926601) (width 0.25) (layer F.Cu) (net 7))
 (segment (start 186.751158 57.926601) (end 186.751158 65.350739) (width 0.25) (layer F.Cu) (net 7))
 (segment (start 189.2752 55.8516) (end 190.5052 55.8516) (width 0.25) (layer F.Cu) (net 7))
 (segment (start 190.5052 55.8516) (end 194.1202 52.2366) (width 0.25) (layer F.Cu) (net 7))
 (segment (start 194.1202 52.2366) (end 194.2752 52.2366) (width 0.25) (layer F.Cu) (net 7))
 (segment (start 187.2752 55.8516) (end 189.2752 55.8516) (width 0.25) (layer F.Cu) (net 7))
 (segment (start 192.95 66.49924) (end 192.95 65.84919) (width 0.25) (layer F.Cu) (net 9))
 (segment (start 191.85081 64.75) (end 191.5 64.75) (width 0.25) (layer F.Cu) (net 9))
 (segment (start 192.95 65.84919) (end 191.85081 64.75) (width 0.25) (layer F.Cu) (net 9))
 (segment (start 192 68.49822) (end 192 70) (width 0.25) (layer F.Cu) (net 11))
 (segment (start 192 70) (end 191.75 70.25) (width 0.25) (layer F.Cu) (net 11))
 (segment (start 191.75 70.25) (end 193.75 70.25) (width 0.25) (layer F.Cu) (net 11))
 (segment (start 188.5 64.96) (end 186.04 64.96) (width 0.25) (layer B.Cu) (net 15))
 (segment (start 186.04 64.96) (end 185.5 65.5) (width 0.25) (layer B.Cu) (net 15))
 (via (at 188.5 64.96) (size 0.6) (drill 0.4) (layers F.Cu B.Cu) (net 15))
 (segment (start 184.45 65.75) (end 185.25 65.75) (width 0.25) (layer F.Cu) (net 15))
 (segment (start 185.25 65.75) (end 185.5 65.5) (width 0.25) (layer F.Cu) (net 15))
 (segment (start 184.45 65.25) (end 185.25 65.25) (width 0.25) (layer F.Cu) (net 15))
 (segment (start 185.25 65.25) (end 185.5 65.5) (width 0.25) (layer F.Cu) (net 15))
 (via (at 185.5 65.5) (size 0.6) (drill 0.4) (layers F.Cu B.Cu) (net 15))
 (segment (start 191.5 63.25) (end 190.21 63.25) (width 0.25) (layer F.Cu) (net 15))
 (segment (start 190.21 63.25) (end 189.299999 64.160001) (width 0.25) (layer F.Cu) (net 15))
 (segment (start 189.299999 64.160001) (end 188.5 64.96) (width 0.25) (layer F.Cu) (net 15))
 (segment (start 175.55 56.7) (end 175.55 58.7748) (width 0.25) (layer F.Cu) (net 13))
 (segment (start 175.55 58.7748) (end 176.952999 60.177799) (width 0.25) (layer F.Cu) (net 13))
 (segment (start 176.952999 60.177799) (end 178.677799 60.177799) (width 0.25) (layer F.Cu) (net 13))
 (segment (start 178.677799 60.177799) (end 179.25 60.75) (width 0.25) (layer F.Cu) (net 13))
 (segment (start 179.25 60.75) (end 179.25 63.75) (width 0.25) (layer F.Cu) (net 13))
 (segment (start 179.25 63.75) (end 179.25 64.75) (width 0.25) (layer F.Cu) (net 13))
 (segment (start 182.55 65.25) (end 181.17 65.25) (width 0.25) (layer F.Cu) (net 13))
 (segment (start 181.17 65.25) (end 180.67 64.75) (width 0.25) (layer F.Cu) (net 13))
 (segment (start 180.67 64.75) (end 179.25 64.75) (width 0.25) (layer F.Cu) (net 13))
 (segment (start 178 64.75) (end 179.25 64.75) (width 0.25) (layer F.Cu) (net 13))
 (segment (start 181.95 51.85) (end 184.0768 51.85) (width 0.25) (layer F.Cu) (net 14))
 (segment (start 184.0768 51.85) (end 186.0752 49.8516) (width 0.25) (layer F.Cu) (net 14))
 (segment (start 186.0752 49.8516) (end 186.2752 49.8516) (width 0.25) (layer F.Cu) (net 14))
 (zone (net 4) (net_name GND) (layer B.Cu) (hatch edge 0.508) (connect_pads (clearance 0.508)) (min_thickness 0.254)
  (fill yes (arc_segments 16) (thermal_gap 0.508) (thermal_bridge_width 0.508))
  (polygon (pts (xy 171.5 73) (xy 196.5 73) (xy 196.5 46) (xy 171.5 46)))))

